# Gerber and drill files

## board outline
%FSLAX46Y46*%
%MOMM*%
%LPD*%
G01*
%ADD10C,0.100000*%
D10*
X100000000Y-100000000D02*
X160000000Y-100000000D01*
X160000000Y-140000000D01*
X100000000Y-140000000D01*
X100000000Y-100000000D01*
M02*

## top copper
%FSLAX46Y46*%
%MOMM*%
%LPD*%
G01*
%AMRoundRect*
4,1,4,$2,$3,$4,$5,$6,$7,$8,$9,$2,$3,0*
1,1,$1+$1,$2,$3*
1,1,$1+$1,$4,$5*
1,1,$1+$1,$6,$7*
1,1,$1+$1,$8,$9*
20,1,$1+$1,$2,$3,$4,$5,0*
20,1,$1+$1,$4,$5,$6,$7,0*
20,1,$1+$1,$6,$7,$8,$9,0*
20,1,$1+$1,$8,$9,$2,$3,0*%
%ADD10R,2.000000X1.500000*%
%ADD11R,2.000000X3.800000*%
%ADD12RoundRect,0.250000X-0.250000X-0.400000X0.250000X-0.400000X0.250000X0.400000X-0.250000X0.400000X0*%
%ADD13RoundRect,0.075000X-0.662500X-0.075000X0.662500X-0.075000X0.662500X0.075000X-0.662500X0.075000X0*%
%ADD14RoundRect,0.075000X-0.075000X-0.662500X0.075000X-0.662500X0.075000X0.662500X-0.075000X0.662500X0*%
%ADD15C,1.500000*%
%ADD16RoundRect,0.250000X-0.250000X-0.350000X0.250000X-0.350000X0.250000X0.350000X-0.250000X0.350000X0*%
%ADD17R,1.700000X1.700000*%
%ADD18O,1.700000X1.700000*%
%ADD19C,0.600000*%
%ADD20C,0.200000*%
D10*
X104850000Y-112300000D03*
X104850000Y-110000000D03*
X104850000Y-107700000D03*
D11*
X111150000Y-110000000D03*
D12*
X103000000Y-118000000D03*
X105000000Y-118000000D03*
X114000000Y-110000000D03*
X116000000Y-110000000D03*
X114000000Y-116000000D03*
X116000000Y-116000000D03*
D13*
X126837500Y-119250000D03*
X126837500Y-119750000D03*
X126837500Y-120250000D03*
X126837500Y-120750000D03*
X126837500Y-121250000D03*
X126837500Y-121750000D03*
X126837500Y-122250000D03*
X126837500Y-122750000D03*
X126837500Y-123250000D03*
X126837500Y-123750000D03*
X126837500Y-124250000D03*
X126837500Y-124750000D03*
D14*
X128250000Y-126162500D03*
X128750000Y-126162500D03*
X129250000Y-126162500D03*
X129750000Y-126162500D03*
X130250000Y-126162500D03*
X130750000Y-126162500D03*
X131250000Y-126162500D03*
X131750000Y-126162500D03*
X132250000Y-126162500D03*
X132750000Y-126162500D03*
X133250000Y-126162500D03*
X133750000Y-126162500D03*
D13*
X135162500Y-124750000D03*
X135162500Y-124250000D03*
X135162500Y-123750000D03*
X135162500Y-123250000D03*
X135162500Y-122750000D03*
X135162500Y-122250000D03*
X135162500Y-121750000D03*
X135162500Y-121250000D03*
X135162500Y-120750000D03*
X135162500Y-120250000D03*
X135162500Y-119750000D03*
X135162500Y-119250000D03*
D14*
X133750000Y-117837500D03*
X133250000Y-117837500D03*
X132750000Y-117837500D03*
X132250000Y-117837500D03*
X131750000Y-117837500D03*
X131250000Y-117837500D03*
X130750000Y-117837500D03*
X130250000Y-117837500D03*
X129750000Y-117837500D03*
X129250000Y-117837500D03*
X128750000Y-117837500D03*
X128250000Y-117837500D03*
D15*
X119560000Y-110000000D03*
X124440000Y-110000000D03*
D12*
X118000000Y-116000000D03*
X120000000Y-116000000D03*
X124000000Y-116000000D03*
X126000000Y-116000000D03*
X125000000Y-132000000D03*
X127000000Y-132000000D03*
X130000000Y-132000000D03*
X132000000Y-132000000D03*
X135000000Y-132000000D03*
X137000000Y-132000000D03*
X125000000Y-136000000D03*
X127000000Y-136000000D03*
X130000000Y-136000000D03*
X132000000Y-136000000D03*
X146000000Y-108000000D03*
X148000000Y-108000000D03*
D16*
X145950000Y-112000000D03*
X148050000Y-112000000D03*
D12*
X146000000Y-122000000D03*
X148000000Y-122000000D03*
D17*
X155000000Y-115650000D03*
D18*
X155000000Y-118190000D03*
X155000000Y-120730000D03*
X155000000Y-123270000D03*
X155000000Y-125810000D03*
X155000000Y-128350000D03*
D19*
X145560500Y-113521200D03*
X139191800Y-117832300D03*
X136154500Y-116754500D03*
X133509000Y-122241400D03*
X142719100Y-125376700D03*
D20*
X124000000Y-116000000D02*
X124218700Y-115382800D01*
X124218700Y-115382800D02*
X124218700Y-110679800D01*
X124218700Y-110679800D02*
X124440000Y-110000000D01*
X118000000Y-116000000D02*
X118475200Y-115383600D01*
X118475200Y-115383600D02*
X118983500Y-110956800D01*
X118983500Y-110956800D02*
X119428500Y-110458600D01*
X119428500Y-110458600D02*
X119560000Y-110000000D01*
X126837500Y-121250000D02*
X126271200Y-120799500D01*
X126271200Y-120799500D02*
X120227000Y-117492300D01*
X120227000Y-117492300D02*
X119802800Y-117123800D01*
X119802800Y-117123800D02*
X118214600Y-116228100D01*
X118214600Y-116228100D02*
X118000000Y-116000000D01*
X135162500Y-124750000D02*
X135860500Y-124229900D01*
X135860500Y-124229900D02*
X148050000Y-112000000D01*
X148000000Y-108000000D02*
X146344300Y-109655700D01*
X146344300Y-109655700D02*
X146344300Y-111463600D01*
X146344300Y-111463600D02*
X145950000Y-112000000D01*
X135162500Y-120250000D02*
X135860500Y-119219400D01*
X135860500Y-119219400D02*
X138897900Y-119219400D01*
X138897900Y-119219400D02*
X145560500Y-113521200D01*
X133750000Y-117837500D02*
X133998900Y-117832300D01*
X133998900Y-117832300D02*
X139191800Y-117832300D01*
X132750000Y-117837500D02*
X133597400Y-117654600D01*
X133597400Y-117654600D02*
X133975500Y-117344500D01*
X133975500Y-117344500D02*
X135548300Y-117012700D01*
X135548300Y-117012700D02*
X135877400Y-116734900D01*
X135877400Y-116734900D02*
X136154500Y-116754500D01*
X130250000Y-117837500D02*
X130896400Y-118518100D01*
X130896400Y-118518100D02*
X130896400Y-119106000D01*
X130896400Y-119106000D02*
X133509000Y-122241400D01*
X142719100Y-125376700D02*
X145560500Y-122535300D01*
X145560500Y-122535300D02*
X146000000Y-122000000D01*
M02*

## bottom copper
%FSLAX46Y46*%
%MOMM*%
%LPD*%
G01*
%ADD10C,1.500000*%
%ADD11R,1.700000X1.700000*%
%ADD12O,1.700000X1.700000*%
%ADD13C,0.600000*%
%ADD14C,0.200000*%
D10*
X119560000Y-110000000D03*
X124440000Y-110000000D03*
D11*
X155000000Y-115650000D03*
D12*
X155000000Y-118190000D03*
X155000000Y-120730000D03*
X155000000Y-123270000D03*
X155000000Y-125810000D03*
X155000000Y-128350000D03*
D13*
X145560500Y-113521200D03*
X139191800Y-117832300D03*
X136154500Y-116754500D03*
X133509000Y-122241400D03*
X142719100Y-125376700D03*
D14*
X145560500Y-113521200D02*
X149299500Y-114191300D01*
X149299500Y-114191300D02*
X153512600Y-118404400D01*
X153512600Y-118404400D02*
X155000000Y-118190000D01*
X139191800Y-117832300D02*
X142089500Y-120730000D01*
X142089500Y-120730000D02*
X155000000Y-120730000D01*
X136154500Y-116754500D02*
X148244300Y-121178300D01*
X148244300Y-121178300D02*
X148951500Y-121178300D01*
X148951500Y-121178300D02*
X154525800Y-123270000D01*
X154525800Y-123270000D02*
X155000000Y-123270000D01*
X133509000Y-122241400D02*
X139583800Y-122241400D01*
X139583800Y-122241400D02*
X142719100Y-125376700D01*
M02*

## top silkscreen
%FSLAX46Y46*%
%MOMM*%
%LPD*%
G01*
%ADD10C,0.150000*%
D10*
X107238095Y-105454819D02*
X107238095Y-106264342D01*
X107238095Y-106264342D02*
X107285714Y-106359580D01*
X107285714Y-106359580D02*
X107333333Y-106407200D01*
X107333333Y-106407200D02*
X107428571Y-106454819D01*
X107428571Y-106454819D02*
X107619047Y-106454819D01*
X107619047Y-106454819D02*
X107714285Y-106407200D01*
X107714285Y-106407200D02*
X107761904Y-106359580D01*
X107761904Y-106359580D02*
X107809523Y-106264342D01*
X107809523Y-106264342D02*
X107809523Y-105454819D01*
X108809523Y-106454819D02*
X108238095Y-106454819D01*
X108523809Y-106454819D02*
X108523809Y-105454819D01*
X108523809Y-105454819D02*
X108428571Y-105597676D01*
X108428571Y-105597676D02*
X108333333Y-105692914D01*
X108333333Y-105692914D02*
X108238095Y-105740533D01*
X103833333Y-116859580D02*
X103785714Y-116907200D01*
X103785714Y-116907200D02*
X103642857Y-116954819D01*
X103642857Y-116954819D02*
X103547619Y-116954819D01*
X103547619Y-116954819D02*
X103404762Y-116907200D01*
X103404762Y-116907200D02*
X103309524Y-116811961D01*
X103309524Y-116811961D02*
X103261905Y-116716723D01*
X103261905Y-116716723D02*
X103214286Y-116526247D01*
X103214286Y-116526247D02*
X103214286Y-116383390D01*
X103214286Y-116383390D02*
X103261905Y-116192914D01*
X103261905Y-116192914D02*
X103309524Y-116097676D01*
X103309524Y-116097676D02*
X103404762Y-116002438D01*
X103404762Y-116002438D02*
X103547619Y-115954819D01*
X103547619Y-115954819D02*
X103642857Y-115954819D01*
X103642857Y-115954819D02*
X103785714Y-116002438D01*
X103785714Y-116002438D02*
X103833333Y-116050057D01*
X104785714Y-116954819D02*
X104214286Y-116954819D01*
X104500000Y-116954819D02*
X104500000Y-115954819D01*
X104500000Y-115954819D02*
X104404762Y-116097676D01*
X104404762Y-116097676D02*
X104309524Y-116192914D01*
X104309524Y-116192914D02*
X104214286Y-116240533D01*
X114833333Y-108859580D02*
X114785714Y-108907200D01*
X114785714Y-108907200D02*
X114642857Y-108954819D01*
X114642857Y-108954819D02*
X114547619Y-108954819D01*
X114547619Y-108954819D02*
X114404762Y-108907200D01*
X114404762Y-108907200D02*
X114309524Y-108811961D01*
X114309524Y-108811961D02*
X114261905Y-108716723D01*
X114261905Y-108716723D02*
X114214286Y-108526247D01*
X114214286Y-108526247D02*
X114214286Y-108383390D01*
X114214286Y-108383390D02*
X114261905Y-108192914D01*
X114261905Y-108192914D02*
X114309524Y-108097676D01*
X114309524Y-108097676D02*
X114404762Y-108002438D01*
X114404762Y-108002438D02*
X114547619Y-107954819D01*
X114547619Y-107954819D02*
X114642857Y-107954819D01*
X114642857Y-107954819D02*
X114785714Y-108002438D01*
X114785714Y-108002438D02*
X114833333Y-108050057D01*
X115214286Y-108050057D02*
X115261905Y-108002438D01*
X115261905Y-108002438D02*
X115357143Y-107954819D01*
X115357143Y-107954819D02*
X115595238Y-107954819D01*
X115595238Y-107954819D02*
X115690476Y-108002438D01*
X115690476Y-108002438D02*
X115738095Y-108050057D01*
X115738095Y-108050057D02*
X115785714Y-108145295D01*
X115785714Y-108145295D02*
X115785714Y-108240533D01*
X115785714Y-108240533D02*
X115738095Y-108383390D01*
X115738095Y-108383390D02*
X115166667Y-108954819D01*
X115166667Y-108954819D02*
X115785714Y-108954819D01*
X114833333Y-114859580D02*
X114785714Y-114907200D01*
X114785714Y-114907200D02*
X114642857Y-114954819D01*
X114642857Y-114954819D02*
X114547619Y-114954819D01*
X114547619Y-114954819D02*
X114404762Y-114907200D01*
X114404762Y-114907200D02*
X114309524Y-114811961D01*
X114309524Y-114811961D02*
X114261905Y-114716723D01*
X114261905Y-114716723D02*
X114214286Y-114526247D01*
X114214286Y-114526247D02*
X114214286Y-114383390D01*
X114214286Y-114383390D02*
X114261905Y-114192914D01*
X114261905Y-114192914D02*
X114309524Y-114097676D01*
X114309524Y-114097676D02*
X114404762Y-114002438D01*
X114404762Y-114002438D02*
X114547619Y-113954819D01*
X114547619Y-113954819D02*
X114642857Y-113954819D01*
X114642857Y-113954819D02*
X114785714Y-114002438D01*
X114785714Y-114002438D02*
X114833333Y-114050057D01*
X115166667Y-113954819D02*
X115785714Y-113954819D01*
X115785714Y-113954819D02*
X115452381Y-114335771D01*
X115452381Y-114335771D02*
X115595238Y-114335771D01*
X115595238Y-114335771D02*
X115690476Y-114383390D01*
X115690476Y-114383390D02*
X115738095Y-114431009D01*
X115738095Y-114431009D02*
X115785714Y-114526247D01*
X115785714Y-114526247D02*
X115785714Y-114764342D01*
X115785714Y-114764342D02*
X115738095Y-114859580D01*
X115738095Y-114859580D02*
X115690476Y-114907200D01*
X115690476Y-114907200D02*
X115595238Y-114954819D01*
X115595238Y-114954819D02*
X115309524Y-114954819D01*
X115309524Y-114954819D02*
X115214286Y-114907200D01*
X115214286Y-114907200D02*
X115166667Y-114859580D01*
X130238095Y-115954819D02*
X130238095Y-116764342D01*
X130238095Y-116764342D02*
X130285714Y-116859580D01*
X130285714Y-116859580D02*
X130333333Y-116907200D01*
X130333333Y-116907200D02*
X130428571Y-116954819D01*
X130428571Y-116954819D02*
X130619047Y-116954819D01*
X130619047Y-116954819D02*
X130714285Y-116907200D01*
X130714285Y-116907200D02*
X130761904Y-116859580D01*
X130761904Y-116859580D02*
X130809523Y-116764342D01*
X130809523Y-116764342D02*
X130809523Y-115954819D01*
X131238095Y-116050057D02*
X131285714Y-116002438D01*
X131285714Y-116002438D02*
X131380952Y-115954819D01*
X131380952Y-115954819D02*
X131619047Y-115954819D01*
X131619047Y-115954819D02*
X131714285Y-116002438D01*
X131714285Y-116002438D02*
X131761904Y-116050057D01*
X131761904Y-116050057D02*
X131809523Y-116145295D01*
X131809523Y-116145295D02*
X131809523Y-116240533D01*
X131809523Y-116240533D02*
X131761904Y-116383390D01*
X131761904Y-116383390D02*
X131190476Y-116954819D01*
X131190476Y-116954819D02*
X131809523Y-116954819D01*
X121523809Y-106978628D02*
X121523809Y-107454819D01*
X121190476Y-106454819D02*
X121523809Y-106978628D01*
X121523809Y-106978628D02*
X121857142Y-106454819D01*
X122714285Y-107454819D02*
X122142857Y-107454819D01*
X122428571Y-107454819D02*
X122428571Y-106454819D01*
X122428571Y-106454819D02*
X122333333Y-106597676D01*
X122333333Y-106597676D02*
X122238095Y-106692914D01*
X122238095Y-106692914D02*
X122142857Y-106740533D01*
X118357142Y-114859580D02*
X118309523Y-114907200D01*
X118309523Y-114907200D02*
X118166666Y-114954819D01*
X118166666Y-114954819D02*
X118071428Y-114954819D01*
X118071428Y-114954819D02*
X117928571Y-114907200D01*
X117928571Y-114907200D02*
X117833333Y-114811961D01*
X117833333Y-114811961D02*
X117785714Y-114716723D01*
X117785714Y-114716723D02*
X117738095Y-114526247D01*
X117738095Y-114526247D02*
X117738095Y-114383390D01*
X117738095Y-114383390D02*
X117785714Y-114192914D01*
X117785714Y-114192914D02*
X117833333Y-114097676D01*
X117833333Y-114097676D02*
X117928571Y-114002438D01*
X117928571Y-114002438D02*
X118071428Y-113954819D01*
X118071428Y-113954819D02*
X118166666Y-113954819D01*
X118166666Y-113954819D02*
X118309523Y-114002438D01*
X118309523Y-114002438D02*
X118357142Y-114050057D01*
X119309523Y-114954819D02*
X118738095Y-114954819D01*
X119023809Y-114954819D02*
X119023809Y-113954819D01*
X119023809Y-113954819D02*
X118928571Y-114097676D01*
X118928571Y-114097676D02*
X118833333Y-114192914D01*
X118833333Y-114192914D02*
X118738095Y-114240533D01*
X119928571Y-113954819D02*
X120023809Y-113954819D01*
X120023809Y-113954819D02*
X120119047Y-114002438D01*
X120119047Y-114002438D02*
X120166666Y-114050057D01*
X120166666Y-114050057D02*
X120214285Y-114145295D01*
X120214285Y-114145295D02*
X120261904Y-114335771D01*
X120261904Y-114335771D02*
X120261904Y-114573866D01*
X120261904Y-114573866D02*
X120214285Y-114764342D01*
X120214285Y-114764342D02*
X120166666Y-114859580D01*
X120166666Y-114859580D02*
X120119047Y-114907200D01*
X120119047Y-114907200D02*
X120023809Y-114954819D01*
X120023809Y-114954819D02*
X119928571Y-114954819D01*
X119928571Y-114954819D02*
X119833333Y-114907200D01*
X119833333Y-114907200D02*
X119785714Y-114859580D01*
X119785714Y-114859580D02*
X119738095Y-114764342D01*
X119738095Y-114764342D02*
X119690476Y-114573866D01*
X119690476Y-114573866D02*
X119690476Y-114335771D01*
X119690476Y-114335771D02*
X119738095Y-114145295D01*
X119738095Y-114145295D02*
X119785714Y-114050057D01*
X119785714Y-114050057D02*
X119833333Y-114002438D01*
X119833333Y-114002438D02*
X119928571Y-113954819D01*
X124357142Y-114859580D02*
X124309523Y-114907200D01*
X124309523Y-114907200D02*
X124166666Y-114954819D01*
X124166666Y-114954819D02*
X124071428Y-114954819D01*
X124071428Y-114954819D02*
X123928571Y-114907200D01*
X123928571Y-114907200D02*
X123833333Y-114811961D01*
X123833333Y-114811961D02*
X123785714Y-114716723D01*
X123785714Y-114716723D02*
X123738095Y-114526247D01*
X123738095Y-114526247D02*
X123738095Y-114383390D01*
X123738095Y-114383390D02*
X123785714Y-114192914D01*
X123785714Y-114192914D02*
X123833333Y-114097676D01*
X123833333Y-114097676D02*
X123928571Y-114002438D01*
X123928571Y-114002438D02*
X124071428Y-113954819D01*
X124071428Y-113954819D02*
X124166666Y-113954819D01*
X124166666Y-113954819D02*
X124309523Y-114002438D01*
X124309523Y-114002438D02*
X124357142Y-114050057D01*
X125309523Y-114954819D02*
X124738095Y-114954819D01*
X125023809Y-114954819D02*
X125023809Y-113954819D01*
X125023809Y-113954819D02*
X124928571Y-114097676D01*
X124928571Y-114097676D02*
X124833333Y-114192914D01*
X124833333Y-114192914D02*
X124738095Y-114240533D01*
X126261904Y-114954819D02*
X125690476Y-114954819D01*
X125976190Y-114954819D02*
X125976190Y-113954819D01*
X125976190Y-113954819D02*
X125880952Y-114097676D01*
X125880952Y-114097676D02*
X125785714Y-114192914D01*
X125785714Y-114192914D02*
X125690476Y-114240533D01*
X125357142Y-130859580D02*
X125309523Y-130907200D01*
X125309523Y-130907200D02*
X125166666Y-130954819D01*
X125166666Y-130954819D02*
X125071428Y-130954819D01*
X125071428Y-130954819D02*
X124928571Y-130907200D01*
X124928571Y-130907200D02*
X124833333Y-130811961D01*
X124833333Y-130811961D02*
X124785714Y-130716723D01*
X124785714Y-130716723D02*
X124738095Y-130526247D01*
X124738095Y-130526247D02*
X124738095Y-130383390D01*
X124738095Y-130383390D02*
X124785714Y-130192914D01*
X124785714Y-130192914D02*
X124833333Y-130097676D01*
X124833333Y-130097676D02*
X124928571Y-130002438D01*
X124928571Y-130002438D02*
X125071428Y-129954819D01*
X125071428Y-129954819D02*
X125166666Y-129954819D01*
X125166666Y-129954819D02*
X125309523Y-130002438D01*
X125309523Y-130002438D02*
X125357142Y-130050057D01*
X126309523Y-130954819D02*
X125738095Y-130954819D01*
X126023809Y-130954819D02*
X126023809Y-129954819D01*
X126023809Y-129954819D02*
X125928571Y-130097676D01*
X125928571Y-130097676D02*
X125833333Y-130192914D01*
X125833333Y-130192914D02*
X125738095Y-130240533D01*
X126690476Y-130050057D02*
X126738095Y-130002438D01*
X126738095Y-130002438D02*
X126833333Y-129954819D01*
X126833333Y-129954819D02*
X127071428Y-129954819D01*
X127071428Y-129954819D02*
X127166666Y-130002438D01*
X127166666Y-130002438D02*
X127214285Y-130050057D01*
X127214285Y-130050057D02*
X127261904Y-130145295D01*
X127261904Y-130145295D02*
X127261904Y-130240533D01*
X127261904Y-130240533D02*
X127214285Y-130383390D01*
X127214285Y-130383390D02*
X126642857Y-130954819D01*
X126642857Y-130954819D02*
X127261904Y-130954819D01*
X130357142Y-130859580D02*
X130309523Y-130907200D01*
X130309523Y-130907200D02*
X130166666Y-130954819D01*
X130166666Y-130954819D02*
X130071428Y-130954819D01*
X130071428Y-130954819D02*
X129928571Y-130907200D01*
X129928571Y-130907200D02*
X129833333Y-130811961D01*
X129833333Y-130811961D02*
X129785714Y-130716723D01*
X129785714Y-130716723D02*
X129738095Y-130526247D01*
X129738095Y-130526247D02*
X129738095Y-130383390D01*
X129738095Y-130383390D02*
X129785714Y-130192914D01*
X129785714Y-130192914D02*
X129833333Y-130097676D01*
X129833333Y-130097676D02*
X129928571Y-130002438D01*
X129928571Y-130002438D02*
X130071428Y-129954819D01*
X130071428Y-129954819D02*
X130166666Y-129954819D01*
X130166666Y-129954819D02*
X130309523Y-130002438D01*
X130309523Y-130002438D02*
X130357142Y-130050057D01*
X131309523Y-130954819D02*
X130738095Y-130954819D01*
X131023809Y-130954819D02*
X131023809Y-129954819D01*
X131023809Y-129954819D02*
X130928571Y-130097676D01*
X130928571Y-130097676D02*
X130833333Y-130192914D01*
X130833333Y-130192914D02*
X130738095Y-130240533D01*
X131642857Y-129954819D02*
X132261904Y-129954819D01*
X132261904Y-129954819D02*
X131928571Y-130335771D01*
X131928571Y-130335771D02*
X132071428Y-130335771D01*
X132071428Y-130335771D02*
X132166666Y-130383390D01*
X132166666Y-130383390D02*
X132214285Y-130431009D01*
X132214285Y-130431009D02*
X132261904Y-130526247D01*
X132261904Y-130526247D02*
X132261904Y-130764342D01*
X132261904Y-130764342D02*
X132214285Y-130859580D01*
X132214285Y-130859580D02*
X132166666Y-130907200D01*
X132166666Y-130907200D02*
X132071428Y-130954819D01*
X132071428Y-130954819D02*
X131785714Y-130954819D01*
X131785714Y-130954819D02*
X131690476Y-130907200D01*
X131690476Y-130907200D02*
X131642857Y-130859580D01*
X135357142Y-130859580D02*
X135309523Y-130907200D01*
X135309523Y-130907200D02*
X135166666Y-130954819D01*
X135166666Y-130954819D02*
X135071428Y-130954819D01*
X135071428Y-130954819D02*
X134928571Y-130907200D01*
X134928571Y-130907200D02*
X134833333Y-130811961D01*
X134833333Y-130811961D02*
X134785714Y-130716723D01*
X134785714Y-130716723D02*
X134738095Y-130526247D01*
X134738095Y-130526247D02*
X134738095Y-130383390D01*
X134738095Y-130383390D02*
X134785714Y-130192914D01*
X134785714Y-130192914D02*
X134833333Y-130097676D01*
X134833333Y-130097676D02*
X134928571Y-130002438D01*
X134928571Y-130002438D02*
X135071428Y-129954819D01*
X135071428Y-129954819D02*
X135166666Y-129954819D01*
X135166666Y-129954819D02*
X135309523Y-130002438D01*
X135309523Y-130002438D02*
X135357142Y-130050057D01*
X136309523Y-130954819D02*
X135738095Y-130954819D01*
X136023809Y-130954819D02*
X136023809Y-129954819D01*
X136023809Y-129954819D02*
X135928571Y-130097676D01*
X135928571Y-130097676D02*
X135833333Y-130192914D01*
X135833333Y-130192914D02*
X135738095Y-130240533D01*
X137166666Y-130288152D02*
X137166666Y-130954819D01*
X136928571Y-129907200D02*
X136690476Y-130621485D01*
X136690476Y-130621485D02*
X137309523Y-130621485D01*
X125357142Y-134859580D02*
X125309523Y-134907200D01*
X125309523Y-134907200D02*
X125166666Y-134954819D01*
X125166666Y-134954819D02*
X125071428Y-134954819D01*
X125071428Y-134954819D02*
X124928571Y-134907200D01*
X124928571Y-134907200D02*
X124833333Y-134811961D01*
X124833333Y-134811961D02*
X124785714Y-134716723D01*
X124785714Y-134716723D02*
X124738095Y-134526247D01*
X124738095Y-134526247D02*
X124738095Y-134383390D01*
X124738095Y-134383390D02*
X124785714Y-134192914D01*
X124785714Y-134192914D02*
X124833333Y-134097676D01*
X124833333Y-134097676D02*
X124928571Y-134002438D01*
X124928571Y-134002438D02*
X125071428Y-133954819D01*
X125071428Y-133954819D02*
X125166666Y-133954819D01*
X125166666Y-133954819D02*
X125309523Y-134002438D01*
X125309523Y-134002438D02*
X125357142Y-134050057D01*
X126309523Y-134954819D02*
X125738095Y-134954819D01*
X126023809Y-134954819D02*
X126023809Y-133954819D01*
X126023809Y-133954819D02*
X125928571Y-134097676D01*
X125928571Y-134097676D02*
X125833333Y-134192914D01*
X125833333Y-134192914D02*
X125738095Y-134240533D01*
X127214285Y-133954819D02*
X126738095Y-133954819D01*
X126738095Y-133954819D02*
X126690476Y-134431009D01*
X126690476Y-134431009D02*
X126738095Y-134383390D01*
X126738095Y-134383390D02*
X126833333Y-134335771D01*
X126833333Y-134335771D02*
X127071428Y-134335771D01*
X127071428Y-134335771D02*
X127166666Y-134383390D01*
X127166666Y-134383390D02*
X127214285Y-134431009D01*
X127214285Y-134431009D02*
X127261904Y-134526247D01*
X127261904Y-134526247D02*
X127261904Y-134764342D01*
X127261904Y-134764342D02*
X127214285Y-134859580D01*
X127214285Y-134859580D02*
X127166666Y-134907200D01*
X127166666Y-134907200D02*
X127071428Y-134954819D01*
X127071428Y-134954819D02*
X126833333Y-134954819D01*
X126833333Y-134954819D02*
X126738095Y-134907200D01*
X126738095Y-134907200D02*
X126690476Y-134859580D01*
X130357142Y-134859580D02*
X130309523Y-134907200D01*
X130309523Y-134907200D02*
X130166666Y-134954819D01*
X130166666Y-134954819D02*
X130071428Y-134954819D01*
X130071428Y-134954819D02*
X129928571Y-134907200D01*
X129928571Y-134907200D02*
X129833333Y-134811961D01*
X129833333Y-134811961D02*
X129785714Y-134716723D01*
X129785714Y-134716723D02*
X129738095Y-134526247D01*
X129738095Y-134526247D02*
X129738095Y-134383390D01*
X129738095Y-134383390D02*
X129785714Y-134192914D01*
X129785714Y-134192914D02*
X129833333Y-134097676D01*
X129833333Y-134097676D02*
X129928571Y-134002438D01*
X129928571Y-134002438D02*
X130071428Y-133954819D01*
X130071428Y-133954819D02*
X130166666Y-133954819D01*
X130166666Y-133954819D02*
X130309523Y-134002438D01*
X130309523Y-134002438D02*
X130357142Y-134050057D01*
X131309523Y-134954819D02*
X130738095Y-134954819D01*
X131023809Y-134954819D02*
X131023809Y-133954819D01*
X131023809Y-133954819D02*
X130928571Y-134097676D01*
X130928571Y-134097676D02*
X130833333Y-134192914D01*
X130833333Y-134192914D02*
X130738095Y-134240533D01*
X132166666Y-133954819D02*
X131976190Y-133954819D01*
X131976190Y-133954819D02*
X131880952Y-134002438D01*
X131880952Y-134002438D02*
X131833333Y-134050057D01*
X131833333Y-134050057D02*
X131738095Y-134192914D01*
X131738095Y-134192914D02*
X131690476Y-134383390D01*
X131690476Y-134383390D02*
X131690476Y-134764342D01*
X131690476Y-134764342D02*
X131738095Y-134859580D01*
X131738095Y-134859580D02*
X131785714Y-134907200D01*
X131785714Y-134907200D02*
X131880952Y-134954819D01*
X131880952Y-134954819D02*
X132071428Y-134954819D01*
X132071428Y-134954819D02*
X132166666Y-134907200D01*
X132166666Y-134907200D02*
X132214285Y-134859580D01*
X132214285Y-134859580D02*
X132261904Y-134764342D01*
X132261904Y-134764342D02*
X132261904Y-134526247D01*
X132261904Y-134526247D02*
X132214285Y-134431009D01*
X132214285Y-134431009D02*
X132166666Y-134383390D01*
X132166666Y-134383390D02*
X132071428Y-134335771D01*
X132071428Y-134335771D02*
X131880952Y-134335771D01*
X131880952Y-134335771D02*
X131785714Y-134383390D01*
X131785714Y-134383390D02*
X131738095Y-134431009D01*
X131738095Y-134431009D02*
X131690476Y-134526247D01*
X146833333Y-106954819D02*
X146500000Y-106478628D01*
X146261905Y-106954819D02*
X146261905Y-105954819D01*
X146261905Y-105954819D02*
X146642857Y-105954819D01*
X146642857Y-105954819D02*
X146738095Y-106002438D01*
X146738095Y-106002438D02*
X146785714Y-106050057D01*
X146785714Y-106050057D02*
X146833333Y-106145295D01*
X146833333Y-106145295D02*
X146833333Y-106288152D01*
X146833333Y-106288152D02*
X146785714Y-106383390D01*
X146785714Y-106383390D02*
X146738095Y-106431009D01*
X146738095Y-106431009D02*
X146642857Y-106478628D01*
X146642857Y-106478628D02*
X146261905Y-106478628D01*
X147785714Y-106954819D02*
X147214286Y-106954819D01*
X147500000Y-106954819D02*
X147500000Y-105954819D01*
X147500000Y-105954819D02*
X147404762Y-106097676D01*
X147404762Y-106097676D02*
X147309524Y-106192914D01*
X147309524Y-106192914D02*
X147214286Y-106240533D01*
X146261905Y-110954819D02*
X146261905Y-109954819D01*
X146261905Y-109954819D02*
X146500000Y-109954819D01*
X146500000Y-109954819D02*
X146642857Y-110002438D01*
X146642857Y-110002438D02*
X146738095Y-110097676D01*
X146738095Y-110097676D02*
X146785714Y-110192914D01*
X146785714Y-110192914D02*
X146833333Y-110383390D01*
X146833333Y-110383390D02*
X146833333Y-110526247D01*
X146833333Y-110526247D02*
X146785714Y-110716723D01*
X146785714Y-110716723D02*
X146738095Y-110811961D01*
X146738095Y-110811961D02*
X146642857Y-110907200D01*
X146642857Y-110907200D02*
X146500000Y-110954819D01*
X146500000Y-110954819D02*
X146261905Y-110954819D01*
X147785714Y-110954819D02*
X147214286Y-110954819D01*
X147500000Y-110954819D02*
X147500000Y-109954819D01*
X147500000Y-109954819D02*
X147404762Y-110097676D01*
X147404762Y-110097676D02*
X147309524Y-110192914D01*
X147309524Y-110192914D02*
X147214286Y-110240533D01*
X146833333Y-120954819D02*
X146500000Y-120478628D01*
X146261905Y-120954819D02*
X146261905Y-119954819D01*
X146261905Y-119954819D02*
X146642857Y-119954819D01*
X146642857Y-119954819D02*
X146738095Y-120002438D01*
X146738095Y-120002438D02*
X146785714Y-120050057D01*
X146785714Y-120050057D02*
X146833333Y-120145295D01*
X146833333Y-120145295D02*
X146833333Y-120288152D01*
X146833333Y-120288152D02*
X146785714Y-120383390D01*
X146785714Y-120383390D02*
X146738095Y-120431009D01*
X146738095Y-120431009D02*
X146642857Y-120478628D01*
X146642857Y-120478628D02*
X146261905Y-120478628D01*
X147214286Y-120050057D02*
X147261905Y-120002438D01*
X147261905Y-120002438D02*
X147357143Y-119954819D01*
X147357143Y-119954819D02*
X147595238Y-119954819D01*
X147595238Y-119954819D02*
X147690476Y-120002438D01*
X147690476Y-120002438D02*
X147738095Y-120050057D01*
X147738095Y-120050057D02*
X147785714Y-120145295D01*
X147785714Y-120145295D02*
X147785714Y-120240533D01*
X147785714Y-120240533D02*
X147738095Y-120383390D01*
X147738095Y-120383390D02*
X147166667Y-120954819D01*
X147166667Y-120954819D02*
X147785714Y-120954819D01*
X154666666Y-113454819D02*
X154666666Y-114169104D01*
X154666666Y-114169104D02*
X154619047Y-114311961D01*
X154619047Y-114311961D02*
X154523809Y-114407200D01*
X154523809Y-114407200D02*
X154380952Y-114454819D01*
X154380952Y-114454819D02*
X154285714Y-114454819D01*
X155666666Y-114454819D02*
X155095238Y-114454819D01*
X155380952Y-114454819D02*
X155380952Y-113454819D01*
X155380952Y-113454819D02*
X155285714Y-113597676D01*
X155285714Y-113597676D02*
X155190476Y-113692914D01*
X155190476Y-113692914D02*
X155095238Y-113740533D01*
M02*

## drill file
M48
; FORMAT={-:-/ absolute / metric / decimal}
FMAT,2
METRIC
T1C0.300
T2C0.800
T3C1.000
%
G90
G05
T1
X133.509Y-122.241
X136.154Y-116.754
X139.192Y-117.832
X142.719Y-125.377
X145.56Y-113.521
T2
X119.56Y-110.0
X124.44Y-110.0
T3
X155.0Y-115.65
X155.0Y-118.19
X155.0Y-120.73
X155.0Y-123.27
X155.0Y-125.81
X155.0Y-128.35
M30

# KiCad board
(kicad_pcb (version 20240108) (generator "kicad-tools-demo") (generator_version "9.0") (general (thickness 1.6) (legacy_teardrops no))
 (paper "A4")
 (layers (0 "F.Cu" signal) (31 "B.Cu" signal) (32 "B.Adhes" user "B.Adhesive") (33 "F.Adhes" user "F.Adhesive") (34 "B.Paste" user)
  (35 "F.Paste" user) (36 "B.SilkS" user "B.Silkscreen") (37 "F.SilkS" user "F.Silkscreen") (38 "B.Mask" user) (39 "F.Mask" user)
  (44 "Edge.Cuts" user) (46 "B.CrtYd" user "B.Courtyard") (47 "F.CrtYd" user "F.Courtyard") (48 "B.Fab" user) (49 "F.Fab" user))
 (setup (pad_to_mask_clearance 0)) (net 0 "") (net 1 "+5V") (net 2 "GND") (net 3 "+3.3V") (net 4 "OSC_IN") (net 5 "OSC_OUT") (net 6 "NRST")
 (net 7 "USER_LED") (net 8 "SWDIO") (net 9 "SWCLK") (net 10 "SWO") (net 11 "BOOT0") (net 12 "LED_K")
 (gr_rect (start 100.0 100.0) (end 160.0 140.0) (stroke (width 0.1) (type default)) (fill none) (layer "Edge.Cuts"))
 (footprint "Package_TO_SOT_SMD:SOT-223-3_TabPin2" (layer "F.Cu") (at 108.0 110.0)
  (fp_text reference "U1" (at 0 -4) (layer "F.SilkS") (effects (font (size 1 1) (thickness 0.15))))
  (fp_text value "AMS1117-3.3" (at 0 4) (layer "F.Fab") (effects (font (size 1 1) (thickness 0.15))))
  (pad "1" smd rect (at -3.15 2.3) (size 2 1.5) (layers "F.Cu" "F.Paste" "F.Mask") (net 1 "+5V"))
  (pad "2" smd rect (at -3.15 0) (size 2 1.5) (layers "F.Cu" "F.Paste" "F.Mask") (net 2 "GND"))
  (pad "3" smd rect (at -3.15 -2.3) (size 2 1.5) (layers "F.Cu" "F.Paste" "F.Mask") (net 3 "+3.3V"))
  (pad "2" smd rect (at 3.15 0) (size 2 3.8) (layers "F.Cu" "F.Paste" "F.Mask") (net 2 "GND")))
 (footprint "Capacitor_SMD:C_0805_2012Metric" (layer "F.Cu") (at 104.0 118.0)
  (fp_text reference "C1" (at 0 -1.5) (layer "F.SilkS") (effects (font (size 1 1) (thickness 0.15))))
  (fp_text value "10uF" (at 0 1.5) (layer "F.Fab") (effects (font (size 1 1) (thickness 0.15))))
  (pad "1" smd roundrect (at -1 0) (size 1.0 1.3) (layers "F.Cu" "F.Paste" "F.Mask") (roundrect_rratio 0.25) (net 1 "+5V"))
  (pad "2" smd roundrect (at 1 0) (size 1.0 1.3) (layers "F.Cu" "F.Paste" "F.Mask") (roundrect_rratio 0.25) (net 2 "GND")))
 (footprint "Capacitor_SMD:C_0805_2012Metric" (layer "F.Cu") (at 115.0 110.0)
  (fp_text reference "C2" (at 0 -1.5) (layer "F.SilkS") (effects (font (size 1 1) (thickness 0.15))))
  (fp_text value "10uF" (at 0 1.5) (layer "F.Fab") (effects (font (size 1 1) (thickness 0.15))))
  (pad "1" smd roundrect (at -1 0) (size 1.0 1.3) (layers "F.Cu" "F.Paste" "F.Mask") (roundrect_rratio 0.25) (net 3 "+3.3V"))
  (pad "2" smd roundrect (at 1 0) (size 1.0 1.3) (layers "F.Cu" "F.Paste" "F.Mask") (roundrect_rratio 0.25) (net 2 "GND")))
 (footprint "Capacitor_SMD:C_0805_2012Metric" (layer "F.Cu") (at 115.0 116.0)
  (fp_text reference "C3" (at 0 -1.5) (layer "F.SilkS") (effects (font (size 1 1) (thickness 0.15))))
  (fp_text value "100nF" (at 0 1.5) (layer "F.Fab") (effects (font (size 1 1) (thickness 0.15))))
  (pad "1" smd roundrect (at -1 0) (size 1.0 1.3) (layers "F.Cu" "F.Paste" "F.Mask") (roundrect_rratio 0.25) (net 3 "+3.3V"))
  (pad "2" smd roundrect (at 1 0) (size 1.0 1.3) (layers "F.Cu" "F.Paste" "F.Mask") (roundrect_rratio 0.25) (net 2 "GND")))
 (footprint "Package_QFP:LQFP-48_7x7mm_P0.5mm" (layer "F.Cu") (at 131.0 122.0)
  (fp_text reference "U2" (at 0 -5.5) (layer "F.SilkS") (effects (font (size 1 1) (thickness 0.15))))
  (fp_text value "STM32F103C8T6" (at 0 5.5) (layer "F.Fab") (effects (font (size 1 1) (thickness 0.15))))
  (pad "1" smd roundrect (at -4.1625 -2.75) (size 1.475 0.3) (layers "F.Cu" "F.Paste" "F.Mask") (roundrect_rratio 0.25) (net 3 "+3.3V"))
  (pad "2" smd roundrect (at -4.1625 -2.25) (size 1.475 0.3) (layers "F.Cu" "F.Paste" "F.Mask") (roundrect_rratio 0.25) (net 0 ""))
  (pad "3" smd roundrect (at -4.1625 -1.75) (size 1.475 0.3) (layers "F.Cu" "F.Paste" "F.Mask") (roundrect_rratio 0.25) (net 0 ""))
  (pad "4" smd roundrect (at -4.1625 -1.25) (size 1.475 0.3) (layers "F.Cu" "F.Paste" "F.Mask") (roundrect_rratio 0.25) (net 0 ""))
  (pad "5" smd roundrect (at -4.1625 -0.75) (size 1.475 0.3) (layers "F.Cu" "F.Paste" "F.Mask") (roundrect_rratio 0.25) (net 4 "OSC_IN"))
  (pad "6" smd roundrect (at -4.1625 -0.25) (size 1.475 0.3) (layers "F.Cu" "F.Paste" "F.Mask") (roundrect_rratio 0.25) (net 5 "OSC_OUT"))
  (pad "7" smd roundrect (at -4.1625 0.25) (size 1.475 0.3) (layers "F.Cu" "F.Paste" "F.Mask") (roundrect_rratio 0.25) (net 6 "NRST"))
  (pad "8" smd roundrect (at -4.1625 0.75) (size 1.475 0.3) (layers "F.Cu" "F.Paste" "F.Mask") (roundrect_rratio 0.25) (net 2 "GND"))
  (pad "9" smd roundrect (at -4.1625 1.25) (size 1.475 0.3) (layers "F.Cu" "F.Paste" "F.Mask") (roundrect_rratio 0.25) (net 3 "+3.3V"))
  (pad "10" smd roundrect (at -4.1625 1.75) (size 1.475 0.3) (layers "F.Cu" "F.Paste" "F.Mask") (roundrect_rratio 0.25) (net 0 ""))
  (pad "11" smd roundrect (at -4.1625 2.25) (size 1.475 0.3) (layers "F.Cu" "F.Paste" "F.Mask") (roundrect_rratio 0.25) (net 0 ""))
  (pad "12" smd roundrect (at -4.1625 2.75) (size 1.475 0.3) (layers "F.Cu" "F.Paste" "F.Mask") (roundrect_rratio 0.25) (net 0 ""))
  (pad "13" smd roundrect (at -2.75 4.1625) (size 0.3 1.475) (layers "F.Cu" "F.Paste" "F.Mask") (roundrect_rratio 0.25) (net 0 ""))
  (pad "14" smd roundrect (at -2.25 4.1625) (size 0.3 1.475) (layers "F.Cu" "F.Paste" "F.Mask") (roundrect_rratio 0.25) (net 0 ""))
  (pad "15" smd roundrect (at -1.75 4.1625) (size 0.3 1.475) (layers "F.Cu" "F.Paste" "F.Mask") (roundrect_rratio 0.25) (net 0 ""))
  (pad "16" smd roundrect (at -1.25 4.1625) (size 0.3 1.475) (layers "F.Cu" "F.Paste" "F.Mask") (roundrect_rratio 0.25) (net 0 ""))
  (pad "17" smd roundrect (at -0.75 4.1625) (size 0.3 1.475) (layers "F.Cu" "F.Paste" "F.Mask") (roundrect_rratio 0.25) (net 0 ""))
  (pad "18" smd roundrect (at -0.25 4.1625) (size 0.3 1.475) (layers "F.Cu" "F.Paste" "F.Mask") (roundrect_rratio 0.25) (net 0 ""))
  (pad "19" smd roundrect (at 0.25 4.1625) (size 0.3 1.475) (layers "F.Cu" "F.Paste" "F.Mask") (roundrect_rratio 0.25) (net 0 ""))
  (pad "20" smd roundrect (at 0.75 4.1625) (size 0.3 1.475) (layers "F.Cu" "F.Paste" "F.Mask") (roundrect_rratio 0.25) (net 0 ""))
  (pad "21" smd roundrect (at 1.25 4.1625) (size 0.3 1.475) (layers "F.Cu" "F.Paste" "F.Mask") (roundrect_rratio 0.25) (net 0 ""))
  (pad "22" smd roundrect (at 1.75 4.1625) (size 0.3 1.475) (layers "F.Cu" "F.Paste" "F.Mask") (roundrect_rratio 0.25) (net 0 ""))
  (pad "23" smd roundrect (at 2.25 4.1625) (size 0.3 1.475) (layers "F.Cu" "F.Paste" "F.Mask") (roundrect_rratio 0.25) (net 2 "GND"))
  (pad "24" smd roundrect (at 2.75 4.1625) (size 0.3 1.475) (layers "F.Cu" "F.Paste" "F.Mask") (roundrect_rratio 0.25) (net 3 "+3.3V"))
  (pad "25" smd roundrect (at 4.1625 2.75) (size 1.475 0.3) (layers "F.Cu" "F.Paste" "F.Mask") (roundrect_rratio 0.25) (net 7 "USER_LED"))
  (pad "26" smd roundrect (at 4.1625 2.25) (size 1.475 0.3) (layers "F.Cu" "F.Paste" "F.Mask") (roundrect_rratio 0.25) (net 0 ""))
  (pad "27" smd roundrect (at 4.1625 1.75) (size 1.475 0.3) (layers "F.Cu" "F.Paste" "F.Mask") (roundrect_rratio 0.25) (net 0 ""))
  (pad "28" smd roundrect (at 4.1625 1.25) (size 1.475 0.3) (layers "F.Cu" "F.Paste" "F.Mask") (roundrect_rratio 0.25) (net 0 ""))
  (pad "29" smd roundrect (at 4.1625 0.75) (size 1.475 0.3) (layers "F.Cu" "F.Paste" "F.Mask") (roundrect_rratio 0.25) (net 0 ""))
  (pad "30" smd roundrect (at 4.1625 0.25) (size 1.475 0.3) (layers "F.Cu" "F.Paste" "F.Mask") (roundrect_rratio 0.25) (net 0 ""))
  (pad "31" smd roundrect (at 4.1625 -0.25) (size 1.475 0.3) (layers "F.Cu" "F.Paste" "F.Mask") (roundrect_rratio 0.25) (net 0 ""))
  (pad "32" smd roundrect (at 4.1625 -0.75) (size 1.475 0.3) (layers "F.Cu" "F.Paste" "F.Mask") (roundrect_rratio 0.25) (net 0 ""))
  (pad "33" smd roundrect (at 4.1625 -1.25) (size 1.475 0.3) (layers "F.Cu" "F.Paste" "F.Mask") (roundrect_rratio 0.25) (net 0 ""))
  (pad "34" smd roundrect (at 4.1625 -1.75) (size 1.475 0.3) (layers "F.Cu" "F.Paste" "F.Mask") (roundrect_rratio 0.25) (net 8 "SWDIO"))
  (pad "35" smd roundrect (at 4.1625 -2.25) (size 1.475 0.3) (layers "F.Cu" "F.Paste" "F.Mask") (roundrect_rratio 0.25) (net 2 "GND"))
  (pad "36" smd roundrect (at 4.1625 -2.75) (size 1.475 0.3) (layers "F.Cu" "F.Paste" "F.Mask") (roundrect_rratio 0.25) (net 3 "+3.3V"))
  (pad "37" smd roundrect (at 2.75 -4.1625) (size 0.3 1.475) (layers "F.Cu" "F.Paste" "F.Mask") (roundrect_rratio 0.25) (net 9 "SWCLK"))
  (pad "38" smd roundrect (at 2.25 -4.1625) (size 0.3 1.475) (layers "F.Cu" "F.Paste" "F.Mask") (roundrect_rratio 0.25) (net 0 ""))
  (pad "39" smd roundrect (at 1.75 -4.1625) (size 0.3 1.475) (layers "F.Cu" "F.Paste" "F.Mask") (roundrect_rratio 0.25) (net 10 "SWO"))
  (pad "40" smd roundrect (at 1.25 -4.1625) (size 0.3 1.475) (layers "F.Cu" "F.Paste" "F.Mask") (roundrect_rratio 0.25) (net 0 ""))
  (pad "41" smd roundrect (at 0.75 -4.1625) (size 0.3 1.475) (layers "F.Cu" "F.Paste" "F.Mask") (roundrect_rratio 0.25) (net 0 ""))
  (pad "42" smd roundrect (at 0.25 -4.1625) (size 0.3 1.475) (layers "F.Cu" "F.Paste" "F.Mask") (roundrect_rratio 0.25) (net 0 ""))
  (pad "43" smd roundrect (at -0.25 -4.1625) (size 0.3 1.475) (layers "F.Cu" "F.Paste" "F.Mask") (roundrect_rratio 0.25) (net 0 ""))
  (pad "44" smd roundrect (at -0.75 -4.1625) (size 0.3 1.475) (layers "F.Cu" "F.Paste" "F.Mask") (roundrect_rratio 0.25) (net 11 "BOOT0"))
  (pad "45" smd roundrect (at -1.25 -4.1625) (size 0.3 1.475) (layers "F.Cu" "F.Paste" "F.Mask") (roundrect_rratio 0.25) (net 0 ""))
  (pad "46" smd roundrect (at -1.75 -4.1625) (size 0.3 1.475) (layers "F.Cu" "F.Paste" "F.Mask") (roundrect_rratio 0.25) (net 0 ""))
  (pad "47" smd roundrect (at -2.25 -4.1625) (size 0.3 1.475) (layers "F.Cu" "F.Paste" "F.Mask") (roundrect_rratio 0.25) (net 2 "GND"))
  (pad "48" smd roundrect (at -2.75 -4.1625) (size 0.3 1.475) (layers "F.Cu" "F.Paste" "F.Mask") (roundrect_rratio 0.25) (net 3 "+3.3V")))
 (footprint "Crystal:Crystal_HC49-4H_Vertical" (layer "F.Cu") (at 122.0 110.0)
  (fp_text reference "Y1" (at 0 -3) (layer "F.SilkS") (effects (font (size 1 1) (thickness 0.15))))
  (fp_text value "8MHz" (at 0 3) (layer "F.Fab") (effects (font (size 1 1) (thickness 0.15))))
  (pad "1" thru_hole circle (at -2.44 0) (size 1.5 1.5) (drill 0.8) (layers "*.Cu" "*.Mask") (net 4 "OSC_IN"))
  (pad "2" thru_hole circle (at 2.44 0) (size 1.5 1.5) (drill 0.8) (layers "*.Cu" "*.Mask") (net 5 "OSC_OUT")))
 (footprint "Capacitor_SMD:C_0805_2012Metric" (layer "F.Cu") (at 119.0 116.0)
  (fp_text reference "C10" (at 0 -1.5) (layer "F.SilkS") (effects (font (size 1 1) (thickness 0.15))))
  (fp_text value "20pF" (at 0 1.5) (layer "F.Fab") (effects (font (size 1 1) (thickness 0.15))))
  (pad "1" smd roundrect (at -1 0) (size 1.0 1.3) (layers "F.Cu" "F.Paste" "F.Mask") (roundrect_rratio 0.25) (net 4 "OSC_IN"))
  (pad "2" smd roundrect (at 1 0) (size 1.0 1.3) (layers "F.Cu" "F.Paste" "F.Mask") (roundrect_rratio 0.25) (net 2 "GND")))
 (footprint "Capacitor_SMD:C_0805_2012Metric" (layer "F.Cu") (at 125.0 116.0)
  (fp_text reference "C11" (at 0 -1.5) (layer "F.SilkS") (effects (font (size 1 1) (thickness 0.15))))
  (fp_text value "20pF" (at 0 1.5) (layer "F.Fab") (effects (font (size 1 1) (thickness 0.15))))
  (pad "1" smd roundrect (at -1 0) (size 1.0 1.3) (layers "F.Cu" "F.Paste" "F.Mask") (roundrect_rratio 0.25) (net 5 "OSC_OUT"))
  (pad "2" smd roundrect (at 1 0) (size 1.0 1.3) (layers "F.Cu" "F.Paste" "F.Mask") (roundrect_rratio 0.25) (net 2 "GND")))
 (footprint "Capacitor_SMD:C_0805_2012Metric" (layer "F.Cu") (at 126.0 132.0)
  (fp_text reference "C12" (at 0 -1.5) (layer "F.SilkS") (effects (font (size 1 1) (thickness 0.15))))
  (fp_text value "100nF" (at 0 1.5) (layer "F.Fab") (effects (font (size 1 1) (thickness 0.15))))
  (pad "1" smd roundrect (at -1 0) (size 1.0 1.3) (layers "F.Cu" "F.Paste" "F.Mask") (roundrect_rratio 0.25) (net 3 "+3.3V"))
  (pad "2" smd roundrect (at 1 0) (size 1.0 1.3) (layers "F.Cu" "F.Paste" "F.Mask") (roundrect_rratio 0.25) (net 2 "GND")))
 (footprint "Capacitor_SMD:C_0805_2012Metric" (layer "F.Cu") (at 131.0 132.0)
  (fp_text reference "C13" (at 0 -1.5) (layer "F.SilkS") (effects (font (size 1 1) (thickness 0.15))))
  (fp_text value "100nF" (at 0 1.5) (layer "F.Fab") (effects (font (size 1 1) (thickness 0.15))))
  (pad "1" smd roundrect (at -1 0) (size 1.0 1.3) (layers "F.Cu" "F.Paste" "F.Mask") (roundrect_rratio 0.25) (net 3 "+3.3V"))
  (pad "2" smd roundrect (at 1 0) (size 1.0 1.3) (layers "F.Cu" "F.Paste" "F.Mask") (roundrect_rratio 0.25) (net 2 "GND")))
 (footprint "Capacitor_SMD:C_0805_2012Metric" (layer "F.Cu") (at 136.0 132.0)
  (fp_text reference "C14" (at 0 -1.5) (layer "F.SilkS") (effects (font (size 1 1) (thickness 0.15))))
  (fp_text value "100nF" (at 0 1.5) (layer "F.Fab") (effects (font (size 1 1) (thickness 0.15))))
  (pad "1" smd roundrect (at -1 0) (size 1.0 1.3) (layers "F.Cu" "F.Paste" "F.Mask") (roundrect_rratio 0.25) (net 3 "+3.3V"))
  (pad "2" smd roundrect (at 1 0) (size 1.0 1.3) (layers "F.Cu" "F.Paste" "F.Mask") (roundrect_rratio 0.25) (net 2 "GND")))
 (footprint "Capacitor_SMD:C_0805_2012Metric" (layer "F.Cu") (at 126.0 136.0)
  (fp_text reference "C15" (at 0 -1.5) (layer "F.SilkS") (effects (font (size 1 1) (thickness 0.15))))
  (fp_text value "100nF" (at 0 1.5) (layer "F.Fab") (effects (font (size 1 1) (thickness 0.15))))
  (pad "1" smd roundrect (at -1 0) (size 1.0 1.3) (layers "F.Cu" "F.Paste" "F.Mask") (roundrect_rratio 0.25) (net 3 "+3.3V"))
  (pad "2" smd roundrect (at 1 0) (size 1.0 1.3) (layers "F.Cu" "F.Paste" "F.Mask") (roundrect_rratio 0.25) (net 2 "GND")))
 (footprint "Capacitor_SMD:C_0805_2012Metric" (layer "F.Cu") (at 131.0 136.0)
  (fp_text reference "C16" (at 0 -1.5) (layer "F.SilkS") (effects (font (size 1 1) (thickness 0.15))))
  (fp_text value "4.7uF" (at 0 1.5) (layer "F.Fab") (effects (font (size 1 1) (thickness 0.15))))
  (pad "1" smd roundrect (at -1 0) (size 1.0 1.3) (layers "F.Cu" "F.Paste" "F.Mask") (roundrect_rratio 0.25) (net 3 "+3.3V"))
  (pad "2" smd roundrect (at 1 0) (size 1.0 1.3) (layers "F.Cu" "F.Paste" "F.Mask") (roundrect_rratio 0.25) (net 2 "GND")))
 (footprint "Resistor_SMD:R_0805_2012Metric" (layer "F.Cu") (at 147.0 108.0)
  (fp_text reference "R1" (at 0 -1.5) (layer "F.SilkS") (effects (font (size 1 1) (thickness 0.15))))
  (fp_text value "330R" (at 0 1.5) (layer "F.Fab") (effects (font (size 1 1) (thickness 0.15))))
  (pad "1" smd roundrect (at -1 0) (size 1.0 1.3) (layers "F.Cu" "F.Paste" "F.Mask") (roundrect_rratio 0.25) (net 3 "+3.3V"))
  (pad "2" smd roundrect (at 1 0) (size 1.0 1.3) (layers "F.Cu" "F.Paste" "F.Mask") (roundrect_rratio 0.25) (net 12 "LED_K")))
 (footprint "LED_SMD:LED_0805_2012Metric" (layer "F.Cu") (at 147.0 112.0)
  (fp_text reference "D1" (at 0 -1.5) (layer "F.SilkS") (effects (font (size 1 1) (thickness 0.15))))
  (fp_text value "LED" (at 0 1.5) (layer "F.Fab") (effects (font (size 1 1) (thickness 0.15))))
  (pad "1" smd roundrect (at -1.05 0) (size 1.0 1.2) (layers "F.Cu" "F.Paste" "F.Mask") (roundrect_rratio 0.25) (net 12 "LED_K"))
  (pad "2" smd roundrect (at 1.05 0) (size 1.0 1.2) (layers "F.Cu" "F.Paste" "F.Mask") (roundrect_rratio 0.25) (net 7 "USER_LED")))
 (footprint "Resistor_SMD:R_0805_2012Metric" (layer "F.Cu") (at 147.0 122.0)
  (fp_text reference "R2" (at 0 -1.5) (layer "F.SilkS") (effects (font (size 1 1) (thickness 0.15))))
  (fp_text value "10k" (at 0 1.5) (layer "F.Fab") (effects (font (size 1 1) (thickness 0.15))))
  (pad "1" smd roundrect (at -1 0) (size 1.0 1.3) (layers "F.Cu" "F.Paste" "F.Mask") (roundrect_rratio 0.25) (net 11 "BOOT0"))
  (pad "2" smd roundrect (at 1 0) (size 1.0 1.3) (layers "F.Cu" "F.Paste" "F.Mask") (roundrect_rratio 0.25) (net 2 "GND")))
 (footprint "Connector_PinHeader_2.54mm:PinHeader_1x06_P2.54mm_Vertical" (layer "F.Cu") (at 155.0 122.0)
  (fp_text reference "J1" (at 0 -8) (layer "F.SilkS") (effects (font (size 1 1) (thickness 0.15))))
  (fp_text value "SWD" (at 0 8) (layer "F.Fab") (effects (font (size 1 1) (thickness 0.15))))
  (pad "1" thru_hole rect (at 0 -6.35) (size 1.7 1.7) (drill 1.0) (layers "*.Cu" "*.Mask") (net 3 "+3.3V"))
  (pad "2" thru_hole oval (at 0 -3.81) (size 1.7 1.7) (drill 1.0) (layers "*.Cu" "*.Mask") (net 8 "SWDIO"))
  (pad "3" thru_hole oval (at 0 -1.27) (size 1.7 1.7) (drill 1.0) (layers "*.Cu" "*.Mask") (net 9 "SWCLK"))
  (pad "4" thru_hole oval (at 0 1.27) (size 1.7 1.7) (drill 1.0) (layers "*.Cu" "*.Mask") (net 10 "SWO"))
  (pad "5" thru_hole oval (at 0 3.81) (size 1.7 1.7) (drill 1.0) (layers "*.Cu" "*.Mask") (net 6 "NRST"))
  (pad "6" thru_hole oval (at 0 6.35) (size 1.7 1.7) (drill 1.0) (layers "*.Cu" "*.Mask") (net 2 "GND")))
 (segment (start 124.0000 116.0000) (end 124.2187 115.3828) (width 0.2) (layer "F.Cu") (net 5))
 (segment (start 124.2187 115.3828) (end 124.2187 110.6798) (width 0.2) (layer "F.Cu") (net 5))
 (segment (start 124.2187 110.6798) (end 124.4400 110.0000) (width 0.2) (layer "F.Cu") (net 5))
 (segment (start 118.0000 116.0000) (end 118.4752 115.3836) (width 0.2) (layer "F.Cu") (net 4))
 (segment (start 118.4752 115.3836) (end 118.9835 110.9568) (width 0.2) (layer "F.Cu") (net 4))
 (segment (start 118.9835 110.9568) (end 119.4285 110.4586) (width 0.2) (layer "F.Cu") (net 4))
 (segment (start 119.4285 110.4586) (end 119.5600 110.0000) (width 0.2) (layer "F.Cu") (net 4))
 (segment (start 126.8375 121.2500) (end 126.2712 120.7995) (width 0.2) (layer "F.Cu") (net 4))
 (segment (start 126.2712 120.7995) (end 120.2270 117.4923) (width 0.2) (layer "F.Cu") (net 4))
 (segment (start 120.2270 117.4923) (end 119.8028 117.1238) (width 0.2) (layer "F.Cu") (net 4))
 (segment (start 119.8028 117.1238) (end 118.2146 116.2281) (width 0.2) (layer "F.Cu") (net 4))
 (segment (start 118.2146 116.2281) (end 118.0000 116.0000) (width 0.2) (layer "F.Cu") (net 4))
 (segment (start 135.1625 124.7500) (end 135.8605 124.2299) (width 0.2) (layer "F.Cu") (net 7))
 (segment (start 135.8605 124.2299) (end 148.0500 112.0000) (width 0.2) (layer "F.Cu") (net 7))
 (segment (start 148.0000 108.0000) (end 146.3443 109.6557) (width 0.2) (layer "F.Cu") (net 12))
 (segment (start 146.3443 109.6557) (end 146.3443 111.4636) (width 0.2) (layer "F.Cu") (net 12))
 (segment (start 146.3443 111.4636) (end 145.9500 112.0000) (width 0.2) (layer "F.Cu") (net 12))
 (segment (start 135.1625 120.2500) (end 135.8605 119.2194) (width 0.2) (layer "F.Cu") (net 8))
 (segment (start 135.8605 119.2194) (end 138.8979 119.2194) (width 0.2) (layer "F.Cu") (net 8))
 (segment (start 138.8979 119.2194) (end 145.5605 113.5212) (width 0.2) (layer "F.Cu") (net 8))
 (segment (start 145.5605 113.5212) (end 149.2995 114.1913) (width 0.2) (layer "B.Cu") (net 8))
 (segment (start 149.2995 114.1913) (end 153.5126 118.4044) (width 0.2) (layer "B.Cu") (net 8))
 (segment (start 153.5126 118.4044) (end 155.0000 118.1900) (width 0.2) (layer "B.Cu") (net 8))
 (via (at 145.5605 113.5212) (size 0.6) (drill 0.3) (layers "F.Cu" "B.Cu") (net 8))
 (segment (start 133.7500 117.8375) (end 133.9989 117.8323) (width 0.2) (layer "F.Cu") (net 9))
 (segment (start 133.9989 117.8323) (end 139.1918 117.8323) (width 0.2) (layer "F.Cu") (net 9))
 (segment (start 139.1918 117.8323) (end 142.0895 120.7300) (width 0.2) (layer "B.Cu") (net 9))
 (segment (start 142.0895 120.7300) (end 155.0000 120.7300) (width 0.2) (layer "B.Cu") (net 9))
 (via (at 139.1918 117.8323) (size 0.6) (drill 0.3) (layers "F.Cu" "B.Cu") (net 9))
 (segment (start 132.7500 117.8375) (end 133.5974 117.6546) (width 0.2) (layer "F.Cu") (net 10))
 (segment (start 133.5974 117.6546) (end 133.9755 117.3445) (width 0.2) (layer "F.Cu") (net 10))
 (segment (start 133.9755 117.3445) (end 135.5483 117.0127) (width 0.2) (layer "F.Cu") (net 10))
 (segment (start 135.5483 117.0127) (end 135.8774 116.7349) (width 0.2) (layer "F.Cu") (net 10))
 (segment (start 135.8774 116.7349) (end 136.1545 116.7545) (width 0.2) (layer "F.Cu") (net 10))
 (segment (start 136.1545 116.7545) (end 148.2443 121.1783) (width 0.2) (layer "B.Cu") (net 10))
 (segment (start 148.2443 121.1783) (end 148.9515 121.1783) (width 0.2) (layer "B.Cu") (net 10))
 (segment (start 148.9515 121.1783) (end 154.5258 123.2700) (width 0.2) (layer "B.Cu") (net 10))
 (segment (start 154.5258 123.2700) (end 155.0000 123.2700) (width 0.2) (layer "B.Cu") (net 10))
 (via (at 136.1545 116.7545) (size 0.6) (drill 0.3) (layers "F.Cu" "B.Cu") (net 10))
 (segment (start 130.2500 117.8375) (end 130.8964 118.5181) (width 0.2) (layer "F.Cu") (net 11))
 (segment (start 130.8964 118.5181) (end 130.8964 119.1060) (width 0.2) (layer "F.Cu") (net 11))
 (segment (start 130.8964 119.1060) (end 133.5090 122.2414) (width 0.2) (layer "F.Cu") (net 11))
 (segment (start 142.7191 125.3767) (end 145.5605 122.5353) (width 0.2) (layer "F.Cu") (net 11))
 (segment (start 145.5605 122.5353) (end 146.0000 122.0000) (width 0.2) (layer "F.Cu") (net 11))
 (segment (start 133.5090 122.2414) (end 139.5838 122.2414) (width 0.2) (layer "B.Cu") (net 11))
 (segment (start 139.5838 122.2414) (end 142.7191 125.3767) (width 0.2) (layer "B.Cu") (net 11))
 (via (at 133.5090 122.2414) (size 0.6) (drill 0.3) (layers "F.Cu" "B.Cu") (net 11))
 (via (at 142.7191 125.3767) (size 0.6) (drill 0.3) (layers "B.Cu" "F.Cu") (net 11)))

